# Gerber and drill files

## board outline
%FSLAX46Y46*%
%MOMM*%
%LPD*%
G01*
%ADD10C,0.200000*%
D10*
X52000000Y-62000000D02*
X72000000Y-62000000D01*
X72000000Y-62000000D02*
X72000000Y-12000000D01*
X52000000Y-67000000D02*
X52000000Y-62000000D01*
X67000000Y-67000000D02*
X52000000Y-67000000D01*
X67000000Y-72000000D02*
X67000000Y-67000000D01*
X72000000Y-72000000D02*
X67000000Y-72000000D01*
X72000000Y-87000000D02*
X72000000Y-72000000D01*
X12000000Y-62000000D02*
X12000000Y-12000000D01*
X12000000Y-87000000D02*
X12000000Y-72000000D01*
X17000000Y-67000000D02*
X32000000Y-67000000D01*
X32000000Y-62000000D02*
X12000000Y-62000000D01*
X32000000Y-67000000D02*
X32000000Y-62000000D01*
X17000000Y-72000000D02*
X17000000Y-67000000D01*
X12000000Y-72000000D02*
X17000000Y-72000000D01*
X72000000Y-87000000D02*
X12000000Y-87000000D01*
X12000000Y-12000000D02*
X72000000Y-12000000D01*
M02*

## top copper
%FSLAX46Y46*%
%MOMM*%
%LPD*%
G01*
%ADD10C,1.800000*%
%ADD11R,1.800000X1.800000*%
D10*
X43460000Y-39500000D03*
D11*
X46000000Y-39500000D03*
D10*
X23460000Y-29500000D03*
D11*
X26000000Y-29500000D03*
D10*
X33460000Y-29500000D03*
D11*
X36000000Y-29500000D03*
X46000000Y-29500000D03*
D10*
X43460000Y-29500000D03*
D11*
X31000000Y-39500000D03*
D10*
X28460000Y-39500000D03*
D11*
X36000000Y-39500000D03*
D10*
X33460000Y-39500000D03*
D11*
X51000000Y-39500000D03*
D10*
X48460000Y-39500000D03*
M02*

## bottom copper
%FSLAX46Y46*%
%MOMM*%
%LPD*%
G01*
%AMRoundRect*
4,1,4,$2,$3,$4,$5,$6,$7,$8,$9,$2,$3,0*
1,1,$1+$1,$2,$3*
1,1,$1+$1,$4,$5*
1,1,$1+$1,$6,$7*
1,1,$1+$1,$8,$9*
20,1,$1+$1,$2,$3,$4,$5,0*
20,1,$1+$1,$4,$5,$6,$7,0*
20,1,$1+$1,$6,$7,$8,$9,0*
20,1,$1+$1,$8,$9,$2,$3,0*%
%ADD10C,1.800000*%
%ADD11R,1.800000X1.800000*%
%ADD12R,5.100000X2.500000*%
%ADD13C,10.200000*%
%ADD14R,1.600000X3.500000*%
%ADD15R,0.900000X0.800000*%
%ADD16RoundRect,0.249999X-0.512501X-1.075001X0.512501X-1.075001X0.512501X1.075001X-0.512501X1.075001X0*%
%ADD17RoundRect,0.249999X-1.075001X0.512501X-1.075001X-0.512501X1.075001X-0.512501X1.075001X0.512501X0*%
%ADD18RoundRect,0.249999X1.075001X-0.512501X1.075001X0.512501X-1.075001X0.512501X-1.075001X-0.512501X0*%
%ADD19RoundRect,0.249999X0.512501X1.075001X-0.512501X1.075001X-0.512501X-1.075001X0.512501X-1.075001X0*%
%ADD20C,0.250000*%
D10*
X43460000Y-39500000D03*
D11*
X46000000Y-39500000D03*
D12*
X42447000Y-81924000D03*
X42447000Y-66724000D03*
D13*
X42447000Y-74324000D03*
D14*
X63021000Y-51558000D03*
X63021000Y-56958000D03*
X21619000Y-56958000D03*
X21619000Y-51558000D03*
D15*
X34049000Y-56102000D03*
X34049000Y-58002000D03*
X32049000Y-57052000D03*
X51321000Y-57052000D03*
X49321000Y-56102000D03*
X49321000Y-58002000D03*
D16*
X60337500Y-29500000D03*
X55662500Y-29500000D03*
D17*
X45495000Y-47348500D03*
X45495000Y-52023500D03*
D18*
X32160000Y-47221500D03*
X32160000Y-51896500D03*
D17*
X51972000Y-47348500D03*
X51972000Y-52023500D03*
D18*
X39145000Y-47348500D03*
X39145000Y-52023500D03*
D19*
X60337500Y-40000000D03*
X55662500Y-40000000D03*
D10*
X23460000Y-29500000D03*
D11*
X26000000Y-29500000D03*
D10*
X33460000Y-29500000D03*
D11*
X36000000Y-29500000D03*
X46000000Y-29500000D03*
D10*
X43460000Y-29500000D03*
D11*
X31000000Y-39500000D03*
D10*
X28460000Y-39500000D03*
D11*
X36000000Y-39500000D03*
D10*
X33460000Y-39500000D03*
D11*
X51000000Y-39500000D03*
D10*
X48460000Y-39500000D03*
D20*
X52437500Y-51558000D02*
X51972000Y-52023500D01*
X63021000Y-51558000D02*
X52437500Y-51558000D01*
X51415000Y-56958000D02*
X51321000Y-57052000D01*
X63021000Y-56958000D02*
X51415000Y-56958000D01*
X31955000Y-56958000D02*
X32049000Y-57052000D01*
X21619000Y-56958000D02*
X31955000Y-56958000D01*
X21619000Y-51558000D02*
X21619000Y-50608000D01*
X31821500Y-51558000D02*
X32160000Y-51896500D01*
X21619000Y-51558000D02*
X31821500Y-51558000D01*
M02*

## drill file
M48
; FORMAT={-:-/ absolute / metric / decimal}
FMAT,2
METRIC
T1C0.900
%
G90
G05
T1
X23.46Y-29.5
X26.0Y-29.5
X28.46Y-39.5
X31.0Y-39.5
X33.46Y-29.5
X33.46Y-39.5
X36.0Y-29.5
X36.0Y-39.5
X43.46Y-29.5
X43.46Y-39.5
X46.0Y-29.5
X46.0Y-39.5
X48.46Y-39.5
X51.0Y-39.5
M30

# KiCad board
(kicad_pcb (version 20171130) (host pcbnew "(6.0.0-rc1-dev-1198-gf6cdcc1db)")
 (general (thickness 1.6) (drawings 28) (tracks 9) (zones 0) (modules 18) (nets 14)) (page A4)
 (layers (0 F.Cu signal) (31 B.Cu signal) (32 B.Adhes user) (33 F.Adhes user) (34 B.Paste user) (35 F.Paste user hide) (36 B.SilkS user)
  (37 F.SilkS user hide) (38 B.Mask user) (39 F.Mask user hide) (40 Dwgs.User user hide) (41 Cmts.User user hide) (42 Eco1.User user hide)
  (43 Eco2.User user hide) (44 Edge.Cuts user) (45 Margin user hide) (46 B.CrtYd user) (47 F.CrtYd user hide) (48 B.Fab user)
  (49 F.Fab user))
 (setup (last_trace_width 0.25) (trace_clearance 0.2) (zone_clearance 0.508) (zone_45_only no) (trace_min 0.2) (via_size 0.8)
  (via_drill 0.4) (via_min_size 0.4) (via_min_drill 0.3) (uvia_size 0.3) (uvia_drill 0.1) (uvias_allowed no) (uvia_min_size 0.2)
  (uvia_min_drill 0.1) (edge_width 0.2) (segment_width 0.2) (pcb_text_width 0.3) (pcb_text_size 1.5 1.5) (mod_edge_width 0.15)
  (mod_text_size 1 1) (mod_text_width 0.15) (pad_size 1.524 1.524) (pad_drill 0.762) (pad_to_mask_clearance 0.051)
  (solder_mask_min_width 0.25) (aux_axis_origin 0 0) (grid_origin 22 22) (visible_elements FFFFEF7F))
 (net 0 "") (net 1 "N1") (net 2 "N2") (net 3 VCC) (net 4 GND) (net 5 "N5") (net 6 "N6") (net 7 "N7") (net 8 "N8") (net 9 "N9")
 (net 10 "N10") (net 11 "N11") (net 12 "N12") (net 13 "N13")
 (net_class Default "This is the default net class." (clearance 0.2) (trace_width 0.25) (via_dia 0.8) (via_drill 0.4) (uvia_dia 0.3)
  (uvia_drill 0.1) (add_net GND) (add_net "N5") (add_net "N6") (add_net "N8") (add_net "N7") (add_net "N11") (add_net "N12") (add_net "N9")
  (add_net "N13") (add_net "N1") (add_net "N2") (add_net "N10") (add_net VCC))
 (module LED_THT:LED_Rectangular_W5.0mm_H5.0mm (layer F.Cu) (at 46 39.5 180)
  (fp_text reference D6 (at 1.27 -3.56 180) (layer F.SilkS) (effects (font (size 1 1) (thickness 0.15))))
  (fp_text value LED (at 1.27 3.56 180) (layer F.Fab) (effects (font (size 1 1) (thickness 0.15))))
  (pad 2 thru_hole circle (at 2.54 0 180) (size 1.8 1.8) (drill 0.9) (layers *.Cu *.Mask) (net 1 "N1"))
  (pad 1 thru_hole rect (at 0 0 180) (size 1.8 1.8) (drill 0.9) (layers *.Cu *.Mask) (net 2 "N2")))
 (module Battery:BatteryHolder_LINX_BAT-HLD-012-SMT (layer B.Cu) (at 42.447 74.324 90)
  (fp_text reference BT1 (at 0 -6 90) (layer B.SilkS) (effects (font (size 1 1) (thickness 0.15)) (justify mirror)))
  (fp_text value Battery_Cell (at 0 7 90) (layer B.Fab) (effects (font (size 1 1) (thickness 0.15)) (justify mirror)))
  (pad 1 smd rect (at -7.6 0 90) (size 2.5 5.1) (layers B.Cu B.Paste B.Mask) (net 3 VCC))
  (pad 1 smd rect (at 7.6 0 90) (size 2.5 5.1) (layers B.Cu B.Paste B.Mask) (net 3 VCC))
  (pad 2 smd circle (at 0 0 90) (size 10.2 10.2) (layers B.Cu B.Paste B.Mask) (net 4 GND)))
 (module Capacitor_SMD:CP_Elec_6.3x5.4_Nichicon (layer B.Cu) (at 63.021 54.258 270)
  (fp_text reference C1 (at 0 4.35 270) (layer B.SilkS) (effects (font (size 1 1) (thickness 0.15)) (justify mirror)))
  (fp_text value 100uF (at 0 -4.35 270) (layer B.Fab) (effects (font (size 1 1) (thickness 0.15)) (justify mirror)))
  (pad 1 smd rect (at -2.7 0 270) (size 3.5 1.6) (layers B.Cu B.Paste B.Mask) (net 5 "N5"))
  (pad 2 smd rect (at 2.7 0 270) (size 3.5 1.6) (layers B.Cu B.Paste B.Mask) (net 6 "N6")))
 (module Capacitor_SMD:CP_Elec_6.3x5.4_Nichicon (layer B.Cu) (at 21.619 54.258 270)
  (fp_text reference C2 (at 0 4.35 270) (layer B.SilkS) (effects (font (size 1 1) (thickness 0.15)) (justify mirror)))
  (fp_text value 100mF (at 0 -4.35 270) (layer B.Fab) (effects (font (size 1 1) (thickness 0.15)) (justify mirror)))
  (pad 2 smd rect (at 2.7 0 270) (size 3.5 1.6) (layers B.Cu B.Paste B.Mask) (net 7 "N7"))
  (pad 1 smd rect (at -2.7 0 270) (size 3.5 1.6) (layers B.Cu B.Paste B.Mask) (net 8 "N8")))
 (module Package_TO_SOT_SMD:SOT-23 (layer B.Cu) (at 33.049 57.052 180)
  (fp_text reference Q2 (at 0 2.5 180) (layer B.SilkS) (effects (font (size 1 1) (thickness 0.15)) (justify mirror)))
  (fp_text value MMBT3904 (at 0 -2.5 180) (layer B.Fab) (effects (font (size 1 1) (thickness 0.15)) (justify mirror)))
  (pad 1 smd rect (at -1 0.95 180) (size 0.9 0.8) (layers B.Cu B.Paste B.Mask) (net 5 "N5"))
  (pad 2 smd rect (at -1 -0.95 180) (size 0.9 0.8) (layers B.Cu B.Paste B.Mask) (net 4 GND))
  (pad 3 smd rect (at 1 0 180) (size 0.9 0.8) (layers B.Cu B.Paste B.Mask) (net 7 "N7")))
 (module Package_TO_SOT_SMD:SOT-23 (layer B.Cu) (at 50.321 57.052)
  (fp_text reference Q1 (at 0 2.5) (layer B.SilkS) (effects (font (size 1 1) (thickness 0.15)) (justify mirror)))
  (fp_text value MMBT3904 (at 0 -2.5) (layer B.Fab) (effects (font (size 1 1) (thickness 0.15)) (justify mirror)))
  (pad 3 smd rect (at 1 0) (size 0.9 0.8) (layers B.Cu B.Paste B.Mask) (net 6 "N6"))
  (pad 2 smd rect (at -1 -0.95) (size 0.9 0.8) (layers B.Cu B.Paste B.Mask) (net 4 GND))
  (pad 1 smd rect (at -1 0.95) (size 0.9 0.8) (layers B.Cu B.Paste B.Mask) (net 8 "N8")))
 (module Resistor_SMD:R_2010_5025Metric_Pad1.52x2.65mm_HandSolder (layer B.Cu) (at 58 29.5)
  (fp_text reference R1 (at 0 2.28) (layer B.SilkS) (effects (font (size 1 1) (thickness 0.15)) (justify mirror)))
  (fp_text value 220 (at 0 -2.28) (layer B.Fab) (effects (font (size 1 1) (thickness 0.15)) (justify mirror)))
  (pad 2 smd roundrect (at 2.3375 0) (size 1.525 2.65) (layers B.Cu B.Paste B.Mask) (roundrect_rratio 0.163934) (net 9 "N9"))
  (pad 1 smd roundrect (at -2.3375 0) (size 1.525 2.65) (layers B.Cu B.Paste B.Mask) (roundrect_rratio 0.163934) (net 6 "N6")))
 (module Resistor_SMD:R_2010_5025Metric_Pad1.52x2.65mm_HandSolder (layer B.Cu) (at 45.495 49.686 270)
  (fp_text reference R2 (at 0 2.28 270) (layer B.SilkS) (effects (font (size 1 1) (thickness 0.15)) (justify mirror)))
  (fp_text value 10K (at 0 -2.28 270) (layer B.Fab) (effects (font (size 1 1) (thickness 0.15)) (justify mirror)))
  (pad 1 smd roundrect (at -2.3375 0 270) (size 1.525 2.65) (layers B.Cu B.Paste B.Mask) (roundrect_rratio 0.163934) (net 6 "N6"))
  (pad 2 smd roundrect (at 2.3375 0 270) (size 1.525 2.65) (layers B.Cu B.Paste B.Mask) (roundrect_rratio 0.163934) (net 3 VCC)))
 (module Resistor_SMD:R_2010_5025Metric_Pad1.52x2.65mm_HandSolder (layer B.Cu) (at 32.16 49.559 90)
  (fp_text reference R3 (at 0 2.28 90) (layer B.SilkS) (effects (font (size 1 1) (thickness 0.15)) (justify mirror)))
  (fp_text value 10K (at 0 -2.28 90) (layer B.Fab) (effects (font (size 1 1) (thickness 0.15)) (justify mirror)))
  (pad 2 smd roundrect (at 2.3375 0 90) (size 1.525 2.65) (layers B.Cu B.Paste B.Mask) (roundrect_rratio 0.163934) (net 3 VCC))
  (pad 1 smd roundrect (at -2.3375 0 90) (size 1.525 2.65) (layers B.Cu B.Paste B.Mask) (roundrect_rratio 0.163934) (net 8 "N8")))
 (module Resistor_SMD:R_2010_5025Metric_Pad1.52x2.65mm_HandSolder (layer B.Cu) (at 51.972 49.686 270)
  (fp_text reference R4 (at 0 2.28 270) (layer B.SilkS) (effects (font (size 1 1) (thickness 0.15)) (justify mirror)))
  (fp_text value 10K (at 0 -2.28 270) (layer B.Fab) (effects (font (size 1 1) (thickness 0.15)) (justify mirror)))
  (pad 1 smd roundrect (at -2.3375 0 270) (size 1.525 2.65) (layers B.Cu B.Paste B.Mask) (roundrect_rratio 0.163934) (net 3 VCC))
  (pad 2 smd roundrect (at 2.3375 0 270) (size 1.525 2.65) (layers B.Cu B.Paste B.Mask) (roundrect_rratio 0.163934) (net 5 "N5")))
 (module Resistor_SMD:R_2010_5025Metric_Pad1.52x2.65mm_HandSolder (layer B.Cu) (at 39.145 49.686 90)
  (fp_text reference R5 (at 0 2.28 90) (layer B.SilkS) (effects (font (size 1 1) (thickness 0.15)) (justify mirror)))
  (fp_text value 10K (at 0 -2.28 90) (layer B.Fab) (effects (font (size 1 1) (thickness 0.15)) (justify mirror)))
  (pad 2 smd roundrect (at 2.3375 0 90) (size 1.525 2.65) (layers B.Cu B.Paste B.Mask) (roundrect_rratio 0.163934) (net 7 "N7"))
  (pad 1 smd roundrect (at -2.3375 0 90) (size 1.525 2.65) (layers B.Cu B.Paste B.Mask) (roundrect_rratio 0.163934) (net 3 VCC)))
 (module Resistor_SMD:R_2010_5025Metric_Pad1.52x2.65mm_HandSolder (layer B.Cu) (at 58 40 180)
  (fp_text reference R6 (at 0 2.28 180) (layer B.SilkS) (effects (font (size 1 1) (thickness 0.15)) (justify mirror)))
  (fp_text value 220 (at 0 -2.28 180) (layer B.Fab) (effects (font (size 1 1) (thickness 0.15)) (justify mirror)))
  (pad 1 smd roundrect (at -2.3375 0 180) (size 1.525 2.65) (layers B.Cu B.Paste B.Mask) (roundrect_rratio 0.163934) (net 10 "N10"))
  (pad 2 smd roundrect (at 2.3375 0 180) (size 1.525 2.65) (layers B.Cu B.Paste B.Mask) (roundrect_rratio 0.163934) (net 7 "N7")))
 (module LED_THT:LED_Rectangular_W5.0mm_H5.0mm (layer F.Cu) (at 26 29.5 180)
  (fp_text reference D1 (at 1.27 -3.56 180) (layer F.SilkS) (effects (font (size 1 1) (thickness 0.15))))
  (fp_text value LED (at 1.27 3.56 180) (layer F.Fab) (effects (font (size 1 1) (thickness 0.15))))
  (pad 2 thru_hole circle (at 2.54 0 180) (size 1.8 1.8) (drill 0.9) (layers *.Cu *.Mask) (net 3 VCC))
  (pad 1 thru_hole rect (at 0 0 180) (size 1.8 1.8) (drill 0.9) (layers *.Cu *.Mask) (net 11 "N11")))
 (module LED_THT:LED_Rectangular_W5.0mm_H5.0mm (layer F.Cu) (at 36 29.5 180)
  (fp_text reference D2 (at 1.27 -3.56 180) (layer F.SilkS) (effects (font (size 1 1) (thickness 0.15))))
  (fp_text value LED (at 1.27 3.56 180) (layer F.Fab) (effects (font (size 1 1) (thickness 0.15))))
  (pad 2 thru_hole circle (at 2.54 0 180) (size 1.8 1.8) (drill 0.9) (layers *.Cu *.Mask) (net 11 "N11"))
  (pad 1 thru_hole rect (at 0 0 180) (size 1.8 1.8) (drill 0.9) (layers *.Cu *.Mask) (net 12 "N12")))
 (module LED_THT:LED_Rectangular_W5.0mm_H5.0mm (layer F.Cu) (at 46 29.5 180)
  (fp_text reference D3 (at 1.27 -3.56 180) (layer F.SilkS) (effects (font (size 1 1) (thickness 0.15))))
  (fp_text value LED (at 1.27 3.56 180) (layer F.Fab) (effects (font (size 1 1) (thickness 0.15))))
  (pad 1 thru_hole rect (at 0 0 180) (size 1.8 1.8) (drill 0.9) (layers *.Cu *.Mask) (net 9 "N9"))
  (pad 2 thru_hole circle (at 2.54 0 180) (size 1.8 1.8) (drill 0.9) (layers *.Cu *.Mask) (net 12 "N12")))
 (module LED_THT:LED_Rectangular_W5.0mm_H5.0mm (layer F.Cu) (at 31 39.5 180)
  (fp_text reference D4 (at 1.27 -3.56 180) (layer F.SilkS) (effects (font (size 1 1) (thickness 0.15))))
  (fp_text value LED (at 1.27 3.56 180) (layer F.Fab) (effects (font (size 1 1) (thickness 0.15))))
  (pad 1 thru_hole rect (at 0 0 180) (size 1.8 1.8) (drill 0.9) (layers *.Cu *.Mask) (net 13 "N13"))
  (pad 2 thru_hole circle (at 2.54 0 180) (size 1.8 1.8) (drill 0.9) (layers *.Cu *.Mask) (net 3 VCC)))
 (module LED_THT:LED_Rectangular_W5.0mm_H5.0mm (layer F.Cu) (at 36 39.5 180)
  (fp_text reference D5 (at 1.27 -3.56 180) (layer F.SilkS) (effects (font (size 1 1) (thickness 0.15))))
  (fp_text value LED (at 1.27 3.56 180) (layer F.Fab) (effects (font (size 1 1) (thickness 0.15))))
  (pad 1 thru_hole rect (at 0 0 180) (size 1.8 1.8) (drill 0.9) (layers *.Cu *.Mask) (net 1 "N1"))
  (pad 2 thru_hole circle (at 2.54 0 180) (size 1.8 1.8) (drill 0.9) (layers *.Cu *.Mask) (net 13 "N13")))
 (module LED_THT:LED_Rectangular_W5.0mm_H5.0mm (layer F.Cu) (at 51 39.5 180)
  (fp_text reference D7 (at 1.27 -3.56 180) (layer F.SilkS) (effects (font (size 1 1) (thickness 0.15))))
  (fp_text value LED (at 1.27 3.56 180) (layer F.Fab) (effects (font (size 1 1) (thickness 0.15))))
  (pad 1 thru_hole rect (at 0 0 180) (size 1.8 1.8) (drill 0.9) (layers *.Cu *.Mask) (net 10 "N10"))
  (pad 2 thru_hole circle (at 2.54 0 180) (size 1.8 1.8) (drill 0.9) (layers *.Cu *.Mask) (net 2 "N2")))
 (gr_line (start 52 62) (end 72 62) (layer Edge.Cuts) (width 0.2))
 (gr_line (start 72 62) (end 72 12) (layer Edge.Cuts) (width 0.2))
 (gr_line (start 52 67) (end 52 62) (layer Edge.Cuts) (width 0.2))
 (gr_line (start 67 67) (end 52 67) (layer Edge.Cuts) (width 0.2))
 (gr_line (start 67 72) (end 67 67) (layer Edge.Cuts) (width 0.2))
 (gr_line (start 72 72) (end 67 72) (layer Edge.Cuts) (width 0.2))
 (gr_line (start 72 87) (end 72 72) (layer Edge.Cuts) (width 0.2))
 (gr_line (start 12 62) (end 12 12) (layer Edge.Cuts) (width 0.2))
 (gr_line (start 12 87) (end 12 72) (layer Edge.Cuts) (width 0.2))
 (gr_line (start 17 67) (end 32 67) (layer Edge.Cuts) (width 0.2))
 (gr_line (start 32 62) (end 12 62) (layer Edge.Cuts) (width 0.2))
 (gr_line (start 32 67) (end 32 62) (layer Edge.Cuts) (width 0.2))
 (gr_line (start 17 72) (end 17 67) (layer Edge.Cuts) (width 0.2))
 (gr_line (start 12 72) (end 17 72) (layer Edge.Cuts) (width 0.2))
 (gr_line (start 72 87) (end 12 87) (layer Edge.Cuts) (width 0.2))
 (gr_line (start 12 12) (end 72 12) (layer Edge.Cuts) (width 0.2))
 (segment (start 52.4375 51.558) (end 51.972 52.0235) (width 0.25) (layer B.Cu) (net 5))
 (segment (start 63.021 51.558) (end 52.4375 51.558) (width 0.25) (layer B.Cu) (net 5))
 (segment (start 51.415 56.958) (end 51.321 57.052) (width 0.25) (layer B.Cu) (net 6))
 (segment (start 63.021 56.958) (end 51.415 56.958) (width 0.25) (layer B.Cu) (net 6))
 (segment (start 31.955 56.958) (end 32.049 57.052) (width 0.25) (layer B.Cu) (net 7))
 (segment (start 21.619 56.958) (end 31.955 56.958) (width 0.25) (layer B.Cu) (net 7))
 (segment (start 21.619 51.558) (end 21.619 50.608) (width 0.25) (layer B.Cu) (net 8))
 (segment (start 31.8215 51.558) (end 32.16 51.8965) (width 0.25) (layer B.Cu) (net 8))
 (segment (start 21.619 51.558) (end 31.8215 51.558) (width 0.25) (layer B.Cu) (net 8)))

